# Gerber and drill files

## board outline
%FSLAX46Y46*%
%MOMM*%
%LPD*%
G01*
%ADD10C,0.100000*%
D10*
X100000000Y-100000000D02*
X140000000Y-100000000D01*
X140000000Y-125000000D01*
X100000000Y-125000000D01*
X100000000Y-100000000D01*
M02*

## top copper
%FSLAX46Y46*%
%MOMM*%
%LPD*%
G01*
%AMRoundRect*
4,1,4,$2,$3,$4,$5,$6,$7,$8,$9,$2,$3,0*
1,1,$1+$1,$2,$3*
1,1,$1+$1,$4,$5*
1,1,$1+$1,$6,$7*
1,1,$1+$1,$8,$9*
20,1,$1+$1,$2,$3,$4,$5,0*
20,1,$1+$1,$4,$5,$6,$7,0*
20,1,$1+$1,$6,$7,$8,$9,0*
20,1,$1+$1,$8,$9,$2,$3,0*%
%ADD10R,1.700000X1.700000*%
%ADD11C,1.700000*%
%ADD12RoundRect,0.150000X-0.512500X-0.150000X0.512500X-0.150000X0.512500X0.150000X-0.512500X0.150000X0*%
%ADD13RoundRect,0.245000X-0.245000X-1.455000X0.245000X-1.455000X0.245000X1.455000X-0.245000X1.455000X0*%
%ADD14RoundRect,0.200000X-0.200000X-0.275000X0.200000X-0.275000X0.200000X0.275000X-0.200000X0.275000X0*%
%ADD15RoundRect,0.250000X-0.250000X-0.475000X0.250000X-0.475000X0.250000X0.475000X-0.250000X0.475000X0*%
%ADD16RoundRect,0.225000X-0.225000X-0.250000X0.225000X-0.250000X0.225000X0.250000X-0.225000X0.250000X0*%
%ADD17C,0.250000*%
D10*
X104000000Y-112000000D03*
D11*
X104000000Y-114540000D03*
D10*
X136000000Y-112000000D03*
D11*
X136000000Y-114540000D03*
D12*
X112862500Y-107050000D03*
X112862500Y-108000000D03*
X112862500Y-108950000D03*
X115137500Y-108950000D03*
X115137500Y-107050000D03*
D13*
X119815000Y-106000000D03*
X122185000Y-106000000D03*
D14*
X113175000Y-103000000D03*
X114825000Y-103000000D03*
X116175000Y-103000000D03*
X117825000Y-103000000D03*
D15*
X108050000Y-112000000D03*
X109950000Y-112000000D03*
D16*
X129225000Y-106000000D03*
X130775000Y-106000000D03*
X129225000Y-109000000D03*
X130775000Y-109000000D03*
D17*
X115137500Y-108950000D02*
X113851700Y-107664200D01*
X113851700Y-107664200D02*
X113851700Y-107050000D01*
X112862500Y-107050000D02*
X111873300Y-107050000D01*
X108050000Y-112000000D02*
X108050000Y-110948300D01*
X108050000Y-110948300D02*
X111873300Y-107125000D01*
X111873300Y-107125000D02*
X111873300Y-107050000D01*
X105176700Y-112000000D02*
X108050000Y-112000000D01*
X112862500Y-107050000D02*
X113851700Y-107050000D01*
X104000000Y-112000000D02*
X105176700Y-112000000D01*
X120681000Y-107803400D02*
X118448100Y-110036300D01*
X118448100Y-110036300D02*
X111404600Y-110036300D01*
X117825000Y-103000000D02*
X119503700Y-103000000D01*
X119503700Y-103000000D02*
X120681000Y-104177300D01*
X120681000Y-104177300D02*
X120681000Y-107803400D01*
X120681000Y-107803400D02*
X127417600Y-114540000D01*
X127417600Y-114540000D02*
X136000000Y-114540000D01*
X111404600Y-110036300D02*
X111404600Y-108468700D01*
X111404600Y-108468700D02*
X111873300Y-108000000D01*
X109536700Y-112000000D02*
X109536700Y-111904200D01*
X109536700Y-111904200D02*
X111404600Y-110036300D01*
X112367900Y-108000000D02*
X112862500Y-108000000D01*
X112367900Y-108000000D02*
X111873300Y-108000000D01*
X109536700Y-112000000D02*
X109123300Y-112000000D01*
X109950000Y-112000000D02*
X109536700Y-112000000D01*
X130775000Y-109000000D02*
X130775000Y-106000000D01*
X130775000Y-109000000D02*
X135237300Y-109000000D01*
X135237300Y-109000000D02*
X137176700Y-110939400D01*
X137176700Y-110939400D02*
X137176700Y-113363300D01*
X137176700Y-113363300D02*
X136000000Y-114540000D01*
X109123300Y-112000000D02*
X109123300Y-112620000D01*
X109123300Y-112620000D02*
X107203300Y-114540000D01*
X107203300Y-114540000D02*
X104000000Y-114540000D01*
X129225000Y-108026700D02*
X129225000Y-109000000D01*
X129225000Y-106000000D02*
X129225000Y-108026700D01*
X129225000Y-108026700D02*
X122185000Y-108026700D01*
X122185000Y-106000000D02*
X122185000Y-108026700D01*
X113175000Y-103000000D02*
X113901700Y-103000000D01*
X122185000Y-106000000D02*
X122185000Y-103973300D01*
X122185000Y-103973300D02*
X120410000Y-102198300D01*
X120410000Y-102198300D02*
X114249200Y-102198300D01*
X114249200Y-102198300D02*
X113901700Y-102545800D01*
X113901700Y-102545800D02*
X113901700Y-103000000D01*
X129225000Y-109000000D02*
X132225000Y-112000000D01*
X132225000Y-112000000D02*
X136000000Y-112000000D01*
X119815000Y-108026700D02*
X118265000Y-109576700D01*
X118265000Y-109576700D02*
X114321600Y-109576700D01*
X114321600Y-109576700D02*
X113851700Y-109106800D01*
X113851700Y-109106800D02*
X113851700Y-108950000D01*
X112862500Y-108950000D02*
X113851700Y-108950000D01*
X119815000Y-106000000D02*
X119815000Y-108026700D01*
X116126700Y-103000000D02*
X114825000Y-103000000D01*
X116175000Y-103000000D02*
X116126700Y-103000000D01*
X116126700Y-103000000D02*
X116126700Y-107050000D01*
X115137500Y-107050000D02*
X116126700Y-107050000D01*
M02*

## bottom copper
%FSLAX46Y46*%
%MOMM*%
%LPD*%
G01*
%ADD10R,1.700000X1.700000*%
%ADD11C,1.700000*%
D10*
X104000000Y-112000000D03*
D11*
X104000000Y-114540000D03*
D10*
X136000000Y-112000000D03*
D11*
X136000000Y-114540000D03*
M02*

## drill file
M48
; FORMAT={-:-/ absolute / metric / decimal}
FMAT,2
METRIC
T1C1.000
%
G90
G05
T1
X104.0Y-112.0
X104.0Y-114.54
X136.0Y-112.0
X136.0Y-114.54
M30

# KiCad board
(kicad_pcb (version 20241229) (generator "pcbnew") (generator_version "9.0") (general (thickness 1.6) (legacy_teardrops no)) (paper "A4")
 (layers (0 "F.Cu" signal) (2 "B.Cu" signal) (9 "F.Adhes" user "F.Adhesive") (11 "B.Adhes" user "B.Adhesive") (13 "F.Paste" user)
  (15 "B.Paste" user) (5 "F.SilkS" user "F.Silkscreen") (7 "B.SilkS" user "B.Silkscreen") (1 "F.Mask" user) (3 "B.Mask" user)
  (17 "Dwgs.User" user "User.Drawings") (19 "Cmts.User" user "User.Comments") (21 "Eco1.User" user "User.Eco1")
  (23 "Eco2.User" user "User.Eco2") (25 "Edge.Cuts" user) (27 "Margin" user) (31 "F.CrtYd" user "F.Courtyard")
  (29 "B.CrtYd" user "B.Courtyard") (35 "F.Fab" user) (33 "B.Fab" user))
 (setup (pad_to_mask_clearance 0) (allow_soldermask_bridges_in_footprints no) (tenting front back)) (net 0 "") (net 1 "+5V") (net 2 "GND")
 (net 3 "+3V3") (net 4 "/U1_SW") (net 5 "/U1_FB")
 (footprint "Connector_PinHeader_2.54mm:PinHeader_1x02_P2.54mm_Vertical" (layer "F.Cu") (at 104 112)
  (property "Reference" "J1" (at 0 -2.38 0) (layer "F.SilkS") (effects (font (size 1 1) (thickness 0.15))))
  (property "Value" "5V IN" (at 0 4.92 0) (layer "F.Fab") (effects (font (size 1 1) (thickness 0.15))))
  (pad "1" thru_hole rect (at 0 0) (size 1.7 1.7) (drill 1) (layers "*.Cu" "*.Mask") (remove_unused_layers no) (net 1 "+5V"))
  (pad "2" thru_hole circle (at 0 2.54) (size 1.7 1.7) (drill 1) (layers "*.Cu" "*.Mask") (remove_unused_layers no) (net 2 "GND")))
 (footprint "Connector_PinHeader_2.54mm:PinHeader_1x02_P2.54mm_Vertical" (layer "F.Cu") (at 136 112)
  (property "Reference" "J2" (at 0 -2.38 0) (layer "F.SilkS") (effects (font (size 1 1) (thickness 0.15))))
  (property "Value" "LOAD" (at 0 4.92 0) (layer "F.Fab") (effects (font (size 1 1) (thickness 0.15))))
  (pad "1" thru_hole rect (at 0 0) (size 1.7 1.7) (drill 1) (layers "*.Cu" "*.Mask") (remove_unused_layers no) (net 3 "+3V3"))
  (pad "2" thru_hole circle (at 0 2.54) (size 1.7 1.7) (drill 1) (layers "*.Cu" "*.Mask") (remove_unused_layers no) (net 2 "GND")))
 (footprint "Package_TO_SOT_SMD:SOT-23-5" (layer "F.Cu") (at 114 108)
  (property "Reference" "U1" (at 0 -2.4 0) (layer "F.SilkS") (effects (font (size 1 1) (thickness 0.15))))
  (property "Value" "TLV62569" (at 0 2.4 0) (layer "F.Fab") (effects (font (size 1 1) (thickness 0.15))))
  (pad "1" smd roundrect (at -1.1375 -0.95) (size 1.325 0.6) (layers "F.Cu" "F.Mask" "F.Paste") (roundrect_rratio 0.25) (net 1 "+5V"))
  (pad "2" smd roundrect (at -1.1375 0) (size 1.325 0.6) (layers "F.Cu" "F.Mask" "F.Paste") (roundrect_rratio 0.25) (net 2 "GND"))
  (pad "3" smd roundrect (at -1.1375 0.95) (size 1.325 0.6) (layers "F.Cu" "F.Mask" "F.Paste") (roundrect_rratio 0.25) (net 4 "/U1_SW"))
  (pad "4" smd roundrect (at 1.1375 0.95) (size 1.325 0.6) (layers "F.Cu" "F.Mask" "F.Paste") (roundrect_rratio 0.25) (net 1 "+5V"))
  (pad "5" smd roundrect (at 1.1375 -0.95) (size 1.325 0.6) (layers "F.Cu" "F.Mask" "F.Paste") (roundrect_rratio 0.25) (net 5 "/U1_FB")))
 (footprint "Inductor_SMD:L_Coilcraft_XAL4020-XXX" (layer "F.Cu") (at 121 106)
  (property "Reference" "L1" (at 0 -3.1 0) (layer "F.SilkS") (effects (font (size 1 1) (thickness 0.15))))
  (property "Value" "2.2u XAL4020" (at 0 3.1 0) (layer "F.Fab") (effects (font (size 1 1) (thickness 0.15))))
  (pad "1" smd roundrect (at -1.185 0) (size 0.98 3.4) (layers "F.Cu" "F.Mask" "F.Paste") (roundrect_rratio 0.25) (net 4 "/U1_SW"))
  (pad "2" smd roundrect (at 1.185 0) (size 0.98 3.4) (layers "F.Cu" "F.Mask" "F.Paste") (roundrect_rratio 0.25) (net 3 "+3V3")))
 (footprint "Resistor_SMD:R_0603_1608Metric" (layer "F.Cu") (at 114 103)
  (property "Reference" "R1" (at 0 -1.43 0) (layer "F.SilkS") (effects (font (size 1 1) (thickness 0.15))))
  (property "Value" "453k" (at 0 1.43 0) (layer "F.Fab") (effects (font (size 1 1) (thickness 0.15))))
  (pad "1" smd roundrect (at -0.825 0) (size 0.8 0.95) (layers "F.Cu" "F.Mask" "F.Paste") (roundrect_rratio 0.25) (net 3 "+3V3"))
  (pad "2" smd roundrect (at 0.825 0) (size 0.8 0.95) (layers "F.Cu" "F.Mask" "F.Paste") (roundrect_rratio 0.25) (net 5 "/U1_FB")))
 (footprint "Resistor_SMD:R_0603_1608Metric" (layer "F.Cu") (at 117 103)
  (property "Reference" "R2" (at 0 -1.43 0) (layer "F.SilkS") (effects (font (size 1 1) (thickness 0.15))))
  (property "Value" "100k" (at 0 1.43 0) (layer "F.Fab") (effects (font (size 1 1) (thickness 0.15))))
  (pad "1" smd roundrect (at -0.825 0) (size 0.8 0.95) (layers "F.Cu" "F.Mask" "F.Paste") (roundrect_rratio 0.25) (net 5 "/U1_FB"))
  (pad "2" smd roundrect (at 0.825 0) (size 0.8 0.95) (layers "F.Cu" "F.Mask" "F.Paste") (roundrect_rratio 0.25) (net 2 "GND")))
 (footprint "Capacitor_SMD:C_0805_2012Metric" (layer "F.Cu") (at 109 112)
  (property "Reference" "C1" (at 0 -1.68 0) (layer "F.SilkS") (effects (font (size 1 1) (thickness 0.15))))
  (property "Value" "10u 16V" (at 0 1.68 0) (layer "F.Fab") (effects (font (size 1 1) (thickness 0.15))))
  (pad "1" smd roundrect (at -0.95 0) (size 1 1.45) (layers "F.Cu" "F.Mask" "F.Paste") (roundrect_rratio 0.25) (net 1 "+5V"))
  (pad "2" smd roundrect (at 0.95 0) (size 1 1.45) (layers "F.Cu" "F.Mask" "F.Paste") (roundrect_rratio 0.25) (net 2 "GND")))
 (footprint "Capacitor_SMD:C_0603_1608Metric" (layer "F.Cu") (at 130 106)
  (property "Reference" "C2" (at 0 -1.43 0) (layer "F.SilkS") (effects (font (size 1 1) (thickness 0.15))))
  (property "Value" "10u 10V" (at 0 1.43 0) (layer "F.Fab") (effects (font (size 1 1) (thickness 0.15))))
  (pad "1" smd roundrect (at -0.775 0) (size 0.9 0.95) (layers "F.Cu" "F.Mask" "F.Paste") (roundrect_rratio 0.25) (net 3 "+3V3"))
  (pad "2" smd roundrect (at 0.775 0) (size 0.9 0.95) (layers "F.Cu" "F.Mask" "F.Paste") (roundrect_rratio 0.25) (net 2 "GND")))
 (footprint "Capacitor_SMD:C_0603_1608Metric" (layer "F.Cu") (at 130 109)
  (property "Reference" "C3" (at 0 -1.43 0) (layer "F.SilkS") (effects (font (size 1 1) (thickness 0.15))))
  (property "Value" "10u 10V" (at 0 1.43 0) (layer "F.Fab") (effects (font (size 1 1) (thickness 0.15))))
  (pad "1" smd roundrect (at -0.775 0) (size 0.9 0.95) (layers "F.Cu" "F.Mask" "F.Paste") (roundrect_rratio 0.25) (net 3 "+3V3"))
  (pad "2" smd roundrect (at 0.775 0) (size 0.9 0.95) (layers "F.Cu" "F.Mask" "F.Paste") (roundrect_rratio 0.25) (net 2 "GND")))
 (gr_rect (start 100 100) (end 140 125) (stroke (width 0.1) (type default)) (fill no) (layer "Edge.Cuts"))
 (segment (start 115.1375 108.95) (end 113.8517 107.6642) (width 0.25) (layer "F.Cu") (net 1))
 (segment (start 113.8517 107.6642) (end 113.8517 107.05) (width 0.25) (layer "F.Cu") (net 1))
 (segment (start 112.8625 107.05) (end 111.8733 107.05) (width 0.25) (layer "F.Cu") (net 1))
 (segment (start 108.05 112) (end 108.05 110.9483) (width 0.25) (layer "F.Cu") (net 1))
 (segment (start 108.05 110.9483) (end 111.8733 107.125) (width 0.25) (layer "F.Cu") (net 1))
 (segment (start 111.8733 107.125) (end 111.8733 107.05) (width 0.25) (layer "F.Cu") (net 1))
 (segment (start 105.1767 112) (end 108.05 112) (width 0.25) (layer "F.Cu") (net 1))
 (segment (start 112.8625 107.05) (end 113.8517 107.05) (width 0.25) (layer "F.Cu") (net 1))
 (segment (start 104 112) (end 105.1767 112) (width 0.25) (layer "F.Cu") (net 1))
 (segment (start 120.681 107.8034) (end 118.4481 110.0363) (width 0.25) (layer "F.Cu") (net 2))
 (segment (start 118.4481 110.0363) (end 111.4046 110.0363) (width 0.25) (layer "F.Cu") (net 2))
 (segment (start 117.825 103) (end 119.5037 103) (width 0.25) (layer "F.Cu") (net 2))
 (segment (start 119.5037 103) (end 120.681 104.1773) (width 0.25) (layer "F.Cu") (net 2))
 (segment (start 120.681 104.1773) (end 120.681 107.8034) (width 0.25) (layer "F.Cu") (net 2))
 (segment (start 120.681 107.8034) (end 127.4176 114.54) (width 0.25) (layer "F.Cu") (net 2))
 (segment (start 127.4176 114.54) (end 136 114.54) (width 0.25) (layer "F.Cu") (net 2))
 (segment (start 111.4046 110.0363) (end 111.4046 108.4687) (width 0.25) (layer "F.Cu") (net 2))
 (segment (start 111.4046 108.4687) (end 111.8733 108) (width 0.25) (layer "F.Cu") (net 2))
 (segment (start 109.5367 112) (end 109.5367 111.9042) (width 0.25) (layer "F.Cu") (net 2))
 (segment (start 109.5367 111.9042) (end 111.4046 110.0363) (width 0.25) (layer "F.Cu") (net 2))
 (segment (start 112.3679 108) (end 112.8625 108) (width 0.25) (layer "F.Cu") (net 2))
 (segment (start 112.3679 108) (end 111.8733 108) (width 0.25) (layer "F.Cu") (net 2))
 (segment (start 109.5367 112) (end 109.1233 112) (width 0.25) (layer "F.Cu") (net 2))
 (segment (start 109.95 112) (end 109.5367 112) (width 0.25) (layer "F.Cu") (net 2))
 (segment (start 130.775 109) (end 130.775 106) (width 0.25) (layer "F.Cu") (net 2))
 (segment (start 130.775 109) (end 135.2373 109) (width 0.25) (layer "F.Cu") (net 2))
 (segment (start 135.2373 109) (end 137.1767 110.9394) (width 0.25) (layer "F.Cu") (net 2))
 (segment (start 137.1767 110.9394) (end 137.1767 113.3633) (width 0.25) (layer "F.Cu") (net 2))
 (segment (start 137.1767 113.3633) (end 136 114.54) (width 0.25) (layer "F.Cu") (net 2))
 (segment (start 109.1233 112) (end 109.1233 112.62) (width 0.25) (layer "F.Cu") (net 2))
 (segment (start 109.1233 112.62) (end 107.2033 114.54) (width 0.25) (layer "F.Cu") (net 2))
 (segment (start 107.2033 114.54) (end 104 114.54) (width 0.25) (layer "F.Cu") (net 2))
 (segment (start 129.225 108.0267) (end 129.225 109) (width 0.25) (layer "F.Cu") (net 3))
 (segment (start 129.225 106) (end 129.225 108.0267) (width 0.25) (layer "F.Cu") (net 3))
 (segment (start 129.225 108.0267) (end 122.185 108.0267) (width 0.25) (layer "F.Cu") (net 3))
 (segment (start 122.185 106) (end 122.185 108.0267) (width 0.25) (layer "F.Cu") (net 3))
 (segment (start 113.175 103) (end 113.9017 103) (width 0.25) (layer "F.Cu") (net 3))
 (segment (start 122.185 106) (end 122.185 103.9733) (width 0.25) (layer "F.Cu") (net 3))
 (segment (start 122.185 103.9733) (end 120.41 102.1983) (width 0.25) (layer "F.Cu") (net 3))
 (segment (start 120.41 102.1983) (end 114.2492 102.1983) (width 0.25) (layer "F.Cu") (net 3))
 (segment (start 114.2492 102.1983) (end 113.9017 102.5458) (width 0.25) (layer "F.Cu") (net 3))
 (segment (start 113.9017 102.5458) (end 113.9017 103) (width 0.25) (layer "F.Cu") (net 3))
 (segment (start 129.225 109) (end 132.225 112) (width 0.25) (layer "F.Cu") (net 3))
 (segment (start 132.225 112) (end 136 112) (width 0.25) (layer "F.Cu") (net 3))
 (segment (start 119.815 108.0267) (end 118.265 109.5767) (width 0.25) (layer "F.Cu") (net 4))
 (segment (start 118.265 109.5767) (end 114.3216 109.5767) (width 0.25) (layer "F.Cu") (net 4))
 (segment (start 114.3216 109.5767) (end 113.8517 109.1068) (width 0.25) (layer "F.Cu") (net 4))
 (segment (start 113.8517 109.1068) (end 113.8517 108.95) (width 0.25) (layer "F.Cu") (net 4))
 (segment (start 112.8625 108.95) (end 113.8517 108.95) (width 0.25) (layer "F.Cu") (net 4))
 (segment (start 119.815 106) (end 119.815 108.0267) (width 0.25) (layer "F.Cu") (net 4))
 (segment (start 116.1267 103) (end 114.825 103) (width 0.25) (layer "F.Cu") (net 5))
 (segment (start 116.175 103) (end 116.1267 103) (width 0.25) (layer "F.Cu") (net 5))
 (segment (start 116.1267 103) (end 116.1267 107.05) (width 0.25) (layer "F.Cu") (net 5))
 (segment (start 115.1375 107.05) (end 116.1267 107.05) (width 0.25) (layer "F.Cu") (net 5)))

